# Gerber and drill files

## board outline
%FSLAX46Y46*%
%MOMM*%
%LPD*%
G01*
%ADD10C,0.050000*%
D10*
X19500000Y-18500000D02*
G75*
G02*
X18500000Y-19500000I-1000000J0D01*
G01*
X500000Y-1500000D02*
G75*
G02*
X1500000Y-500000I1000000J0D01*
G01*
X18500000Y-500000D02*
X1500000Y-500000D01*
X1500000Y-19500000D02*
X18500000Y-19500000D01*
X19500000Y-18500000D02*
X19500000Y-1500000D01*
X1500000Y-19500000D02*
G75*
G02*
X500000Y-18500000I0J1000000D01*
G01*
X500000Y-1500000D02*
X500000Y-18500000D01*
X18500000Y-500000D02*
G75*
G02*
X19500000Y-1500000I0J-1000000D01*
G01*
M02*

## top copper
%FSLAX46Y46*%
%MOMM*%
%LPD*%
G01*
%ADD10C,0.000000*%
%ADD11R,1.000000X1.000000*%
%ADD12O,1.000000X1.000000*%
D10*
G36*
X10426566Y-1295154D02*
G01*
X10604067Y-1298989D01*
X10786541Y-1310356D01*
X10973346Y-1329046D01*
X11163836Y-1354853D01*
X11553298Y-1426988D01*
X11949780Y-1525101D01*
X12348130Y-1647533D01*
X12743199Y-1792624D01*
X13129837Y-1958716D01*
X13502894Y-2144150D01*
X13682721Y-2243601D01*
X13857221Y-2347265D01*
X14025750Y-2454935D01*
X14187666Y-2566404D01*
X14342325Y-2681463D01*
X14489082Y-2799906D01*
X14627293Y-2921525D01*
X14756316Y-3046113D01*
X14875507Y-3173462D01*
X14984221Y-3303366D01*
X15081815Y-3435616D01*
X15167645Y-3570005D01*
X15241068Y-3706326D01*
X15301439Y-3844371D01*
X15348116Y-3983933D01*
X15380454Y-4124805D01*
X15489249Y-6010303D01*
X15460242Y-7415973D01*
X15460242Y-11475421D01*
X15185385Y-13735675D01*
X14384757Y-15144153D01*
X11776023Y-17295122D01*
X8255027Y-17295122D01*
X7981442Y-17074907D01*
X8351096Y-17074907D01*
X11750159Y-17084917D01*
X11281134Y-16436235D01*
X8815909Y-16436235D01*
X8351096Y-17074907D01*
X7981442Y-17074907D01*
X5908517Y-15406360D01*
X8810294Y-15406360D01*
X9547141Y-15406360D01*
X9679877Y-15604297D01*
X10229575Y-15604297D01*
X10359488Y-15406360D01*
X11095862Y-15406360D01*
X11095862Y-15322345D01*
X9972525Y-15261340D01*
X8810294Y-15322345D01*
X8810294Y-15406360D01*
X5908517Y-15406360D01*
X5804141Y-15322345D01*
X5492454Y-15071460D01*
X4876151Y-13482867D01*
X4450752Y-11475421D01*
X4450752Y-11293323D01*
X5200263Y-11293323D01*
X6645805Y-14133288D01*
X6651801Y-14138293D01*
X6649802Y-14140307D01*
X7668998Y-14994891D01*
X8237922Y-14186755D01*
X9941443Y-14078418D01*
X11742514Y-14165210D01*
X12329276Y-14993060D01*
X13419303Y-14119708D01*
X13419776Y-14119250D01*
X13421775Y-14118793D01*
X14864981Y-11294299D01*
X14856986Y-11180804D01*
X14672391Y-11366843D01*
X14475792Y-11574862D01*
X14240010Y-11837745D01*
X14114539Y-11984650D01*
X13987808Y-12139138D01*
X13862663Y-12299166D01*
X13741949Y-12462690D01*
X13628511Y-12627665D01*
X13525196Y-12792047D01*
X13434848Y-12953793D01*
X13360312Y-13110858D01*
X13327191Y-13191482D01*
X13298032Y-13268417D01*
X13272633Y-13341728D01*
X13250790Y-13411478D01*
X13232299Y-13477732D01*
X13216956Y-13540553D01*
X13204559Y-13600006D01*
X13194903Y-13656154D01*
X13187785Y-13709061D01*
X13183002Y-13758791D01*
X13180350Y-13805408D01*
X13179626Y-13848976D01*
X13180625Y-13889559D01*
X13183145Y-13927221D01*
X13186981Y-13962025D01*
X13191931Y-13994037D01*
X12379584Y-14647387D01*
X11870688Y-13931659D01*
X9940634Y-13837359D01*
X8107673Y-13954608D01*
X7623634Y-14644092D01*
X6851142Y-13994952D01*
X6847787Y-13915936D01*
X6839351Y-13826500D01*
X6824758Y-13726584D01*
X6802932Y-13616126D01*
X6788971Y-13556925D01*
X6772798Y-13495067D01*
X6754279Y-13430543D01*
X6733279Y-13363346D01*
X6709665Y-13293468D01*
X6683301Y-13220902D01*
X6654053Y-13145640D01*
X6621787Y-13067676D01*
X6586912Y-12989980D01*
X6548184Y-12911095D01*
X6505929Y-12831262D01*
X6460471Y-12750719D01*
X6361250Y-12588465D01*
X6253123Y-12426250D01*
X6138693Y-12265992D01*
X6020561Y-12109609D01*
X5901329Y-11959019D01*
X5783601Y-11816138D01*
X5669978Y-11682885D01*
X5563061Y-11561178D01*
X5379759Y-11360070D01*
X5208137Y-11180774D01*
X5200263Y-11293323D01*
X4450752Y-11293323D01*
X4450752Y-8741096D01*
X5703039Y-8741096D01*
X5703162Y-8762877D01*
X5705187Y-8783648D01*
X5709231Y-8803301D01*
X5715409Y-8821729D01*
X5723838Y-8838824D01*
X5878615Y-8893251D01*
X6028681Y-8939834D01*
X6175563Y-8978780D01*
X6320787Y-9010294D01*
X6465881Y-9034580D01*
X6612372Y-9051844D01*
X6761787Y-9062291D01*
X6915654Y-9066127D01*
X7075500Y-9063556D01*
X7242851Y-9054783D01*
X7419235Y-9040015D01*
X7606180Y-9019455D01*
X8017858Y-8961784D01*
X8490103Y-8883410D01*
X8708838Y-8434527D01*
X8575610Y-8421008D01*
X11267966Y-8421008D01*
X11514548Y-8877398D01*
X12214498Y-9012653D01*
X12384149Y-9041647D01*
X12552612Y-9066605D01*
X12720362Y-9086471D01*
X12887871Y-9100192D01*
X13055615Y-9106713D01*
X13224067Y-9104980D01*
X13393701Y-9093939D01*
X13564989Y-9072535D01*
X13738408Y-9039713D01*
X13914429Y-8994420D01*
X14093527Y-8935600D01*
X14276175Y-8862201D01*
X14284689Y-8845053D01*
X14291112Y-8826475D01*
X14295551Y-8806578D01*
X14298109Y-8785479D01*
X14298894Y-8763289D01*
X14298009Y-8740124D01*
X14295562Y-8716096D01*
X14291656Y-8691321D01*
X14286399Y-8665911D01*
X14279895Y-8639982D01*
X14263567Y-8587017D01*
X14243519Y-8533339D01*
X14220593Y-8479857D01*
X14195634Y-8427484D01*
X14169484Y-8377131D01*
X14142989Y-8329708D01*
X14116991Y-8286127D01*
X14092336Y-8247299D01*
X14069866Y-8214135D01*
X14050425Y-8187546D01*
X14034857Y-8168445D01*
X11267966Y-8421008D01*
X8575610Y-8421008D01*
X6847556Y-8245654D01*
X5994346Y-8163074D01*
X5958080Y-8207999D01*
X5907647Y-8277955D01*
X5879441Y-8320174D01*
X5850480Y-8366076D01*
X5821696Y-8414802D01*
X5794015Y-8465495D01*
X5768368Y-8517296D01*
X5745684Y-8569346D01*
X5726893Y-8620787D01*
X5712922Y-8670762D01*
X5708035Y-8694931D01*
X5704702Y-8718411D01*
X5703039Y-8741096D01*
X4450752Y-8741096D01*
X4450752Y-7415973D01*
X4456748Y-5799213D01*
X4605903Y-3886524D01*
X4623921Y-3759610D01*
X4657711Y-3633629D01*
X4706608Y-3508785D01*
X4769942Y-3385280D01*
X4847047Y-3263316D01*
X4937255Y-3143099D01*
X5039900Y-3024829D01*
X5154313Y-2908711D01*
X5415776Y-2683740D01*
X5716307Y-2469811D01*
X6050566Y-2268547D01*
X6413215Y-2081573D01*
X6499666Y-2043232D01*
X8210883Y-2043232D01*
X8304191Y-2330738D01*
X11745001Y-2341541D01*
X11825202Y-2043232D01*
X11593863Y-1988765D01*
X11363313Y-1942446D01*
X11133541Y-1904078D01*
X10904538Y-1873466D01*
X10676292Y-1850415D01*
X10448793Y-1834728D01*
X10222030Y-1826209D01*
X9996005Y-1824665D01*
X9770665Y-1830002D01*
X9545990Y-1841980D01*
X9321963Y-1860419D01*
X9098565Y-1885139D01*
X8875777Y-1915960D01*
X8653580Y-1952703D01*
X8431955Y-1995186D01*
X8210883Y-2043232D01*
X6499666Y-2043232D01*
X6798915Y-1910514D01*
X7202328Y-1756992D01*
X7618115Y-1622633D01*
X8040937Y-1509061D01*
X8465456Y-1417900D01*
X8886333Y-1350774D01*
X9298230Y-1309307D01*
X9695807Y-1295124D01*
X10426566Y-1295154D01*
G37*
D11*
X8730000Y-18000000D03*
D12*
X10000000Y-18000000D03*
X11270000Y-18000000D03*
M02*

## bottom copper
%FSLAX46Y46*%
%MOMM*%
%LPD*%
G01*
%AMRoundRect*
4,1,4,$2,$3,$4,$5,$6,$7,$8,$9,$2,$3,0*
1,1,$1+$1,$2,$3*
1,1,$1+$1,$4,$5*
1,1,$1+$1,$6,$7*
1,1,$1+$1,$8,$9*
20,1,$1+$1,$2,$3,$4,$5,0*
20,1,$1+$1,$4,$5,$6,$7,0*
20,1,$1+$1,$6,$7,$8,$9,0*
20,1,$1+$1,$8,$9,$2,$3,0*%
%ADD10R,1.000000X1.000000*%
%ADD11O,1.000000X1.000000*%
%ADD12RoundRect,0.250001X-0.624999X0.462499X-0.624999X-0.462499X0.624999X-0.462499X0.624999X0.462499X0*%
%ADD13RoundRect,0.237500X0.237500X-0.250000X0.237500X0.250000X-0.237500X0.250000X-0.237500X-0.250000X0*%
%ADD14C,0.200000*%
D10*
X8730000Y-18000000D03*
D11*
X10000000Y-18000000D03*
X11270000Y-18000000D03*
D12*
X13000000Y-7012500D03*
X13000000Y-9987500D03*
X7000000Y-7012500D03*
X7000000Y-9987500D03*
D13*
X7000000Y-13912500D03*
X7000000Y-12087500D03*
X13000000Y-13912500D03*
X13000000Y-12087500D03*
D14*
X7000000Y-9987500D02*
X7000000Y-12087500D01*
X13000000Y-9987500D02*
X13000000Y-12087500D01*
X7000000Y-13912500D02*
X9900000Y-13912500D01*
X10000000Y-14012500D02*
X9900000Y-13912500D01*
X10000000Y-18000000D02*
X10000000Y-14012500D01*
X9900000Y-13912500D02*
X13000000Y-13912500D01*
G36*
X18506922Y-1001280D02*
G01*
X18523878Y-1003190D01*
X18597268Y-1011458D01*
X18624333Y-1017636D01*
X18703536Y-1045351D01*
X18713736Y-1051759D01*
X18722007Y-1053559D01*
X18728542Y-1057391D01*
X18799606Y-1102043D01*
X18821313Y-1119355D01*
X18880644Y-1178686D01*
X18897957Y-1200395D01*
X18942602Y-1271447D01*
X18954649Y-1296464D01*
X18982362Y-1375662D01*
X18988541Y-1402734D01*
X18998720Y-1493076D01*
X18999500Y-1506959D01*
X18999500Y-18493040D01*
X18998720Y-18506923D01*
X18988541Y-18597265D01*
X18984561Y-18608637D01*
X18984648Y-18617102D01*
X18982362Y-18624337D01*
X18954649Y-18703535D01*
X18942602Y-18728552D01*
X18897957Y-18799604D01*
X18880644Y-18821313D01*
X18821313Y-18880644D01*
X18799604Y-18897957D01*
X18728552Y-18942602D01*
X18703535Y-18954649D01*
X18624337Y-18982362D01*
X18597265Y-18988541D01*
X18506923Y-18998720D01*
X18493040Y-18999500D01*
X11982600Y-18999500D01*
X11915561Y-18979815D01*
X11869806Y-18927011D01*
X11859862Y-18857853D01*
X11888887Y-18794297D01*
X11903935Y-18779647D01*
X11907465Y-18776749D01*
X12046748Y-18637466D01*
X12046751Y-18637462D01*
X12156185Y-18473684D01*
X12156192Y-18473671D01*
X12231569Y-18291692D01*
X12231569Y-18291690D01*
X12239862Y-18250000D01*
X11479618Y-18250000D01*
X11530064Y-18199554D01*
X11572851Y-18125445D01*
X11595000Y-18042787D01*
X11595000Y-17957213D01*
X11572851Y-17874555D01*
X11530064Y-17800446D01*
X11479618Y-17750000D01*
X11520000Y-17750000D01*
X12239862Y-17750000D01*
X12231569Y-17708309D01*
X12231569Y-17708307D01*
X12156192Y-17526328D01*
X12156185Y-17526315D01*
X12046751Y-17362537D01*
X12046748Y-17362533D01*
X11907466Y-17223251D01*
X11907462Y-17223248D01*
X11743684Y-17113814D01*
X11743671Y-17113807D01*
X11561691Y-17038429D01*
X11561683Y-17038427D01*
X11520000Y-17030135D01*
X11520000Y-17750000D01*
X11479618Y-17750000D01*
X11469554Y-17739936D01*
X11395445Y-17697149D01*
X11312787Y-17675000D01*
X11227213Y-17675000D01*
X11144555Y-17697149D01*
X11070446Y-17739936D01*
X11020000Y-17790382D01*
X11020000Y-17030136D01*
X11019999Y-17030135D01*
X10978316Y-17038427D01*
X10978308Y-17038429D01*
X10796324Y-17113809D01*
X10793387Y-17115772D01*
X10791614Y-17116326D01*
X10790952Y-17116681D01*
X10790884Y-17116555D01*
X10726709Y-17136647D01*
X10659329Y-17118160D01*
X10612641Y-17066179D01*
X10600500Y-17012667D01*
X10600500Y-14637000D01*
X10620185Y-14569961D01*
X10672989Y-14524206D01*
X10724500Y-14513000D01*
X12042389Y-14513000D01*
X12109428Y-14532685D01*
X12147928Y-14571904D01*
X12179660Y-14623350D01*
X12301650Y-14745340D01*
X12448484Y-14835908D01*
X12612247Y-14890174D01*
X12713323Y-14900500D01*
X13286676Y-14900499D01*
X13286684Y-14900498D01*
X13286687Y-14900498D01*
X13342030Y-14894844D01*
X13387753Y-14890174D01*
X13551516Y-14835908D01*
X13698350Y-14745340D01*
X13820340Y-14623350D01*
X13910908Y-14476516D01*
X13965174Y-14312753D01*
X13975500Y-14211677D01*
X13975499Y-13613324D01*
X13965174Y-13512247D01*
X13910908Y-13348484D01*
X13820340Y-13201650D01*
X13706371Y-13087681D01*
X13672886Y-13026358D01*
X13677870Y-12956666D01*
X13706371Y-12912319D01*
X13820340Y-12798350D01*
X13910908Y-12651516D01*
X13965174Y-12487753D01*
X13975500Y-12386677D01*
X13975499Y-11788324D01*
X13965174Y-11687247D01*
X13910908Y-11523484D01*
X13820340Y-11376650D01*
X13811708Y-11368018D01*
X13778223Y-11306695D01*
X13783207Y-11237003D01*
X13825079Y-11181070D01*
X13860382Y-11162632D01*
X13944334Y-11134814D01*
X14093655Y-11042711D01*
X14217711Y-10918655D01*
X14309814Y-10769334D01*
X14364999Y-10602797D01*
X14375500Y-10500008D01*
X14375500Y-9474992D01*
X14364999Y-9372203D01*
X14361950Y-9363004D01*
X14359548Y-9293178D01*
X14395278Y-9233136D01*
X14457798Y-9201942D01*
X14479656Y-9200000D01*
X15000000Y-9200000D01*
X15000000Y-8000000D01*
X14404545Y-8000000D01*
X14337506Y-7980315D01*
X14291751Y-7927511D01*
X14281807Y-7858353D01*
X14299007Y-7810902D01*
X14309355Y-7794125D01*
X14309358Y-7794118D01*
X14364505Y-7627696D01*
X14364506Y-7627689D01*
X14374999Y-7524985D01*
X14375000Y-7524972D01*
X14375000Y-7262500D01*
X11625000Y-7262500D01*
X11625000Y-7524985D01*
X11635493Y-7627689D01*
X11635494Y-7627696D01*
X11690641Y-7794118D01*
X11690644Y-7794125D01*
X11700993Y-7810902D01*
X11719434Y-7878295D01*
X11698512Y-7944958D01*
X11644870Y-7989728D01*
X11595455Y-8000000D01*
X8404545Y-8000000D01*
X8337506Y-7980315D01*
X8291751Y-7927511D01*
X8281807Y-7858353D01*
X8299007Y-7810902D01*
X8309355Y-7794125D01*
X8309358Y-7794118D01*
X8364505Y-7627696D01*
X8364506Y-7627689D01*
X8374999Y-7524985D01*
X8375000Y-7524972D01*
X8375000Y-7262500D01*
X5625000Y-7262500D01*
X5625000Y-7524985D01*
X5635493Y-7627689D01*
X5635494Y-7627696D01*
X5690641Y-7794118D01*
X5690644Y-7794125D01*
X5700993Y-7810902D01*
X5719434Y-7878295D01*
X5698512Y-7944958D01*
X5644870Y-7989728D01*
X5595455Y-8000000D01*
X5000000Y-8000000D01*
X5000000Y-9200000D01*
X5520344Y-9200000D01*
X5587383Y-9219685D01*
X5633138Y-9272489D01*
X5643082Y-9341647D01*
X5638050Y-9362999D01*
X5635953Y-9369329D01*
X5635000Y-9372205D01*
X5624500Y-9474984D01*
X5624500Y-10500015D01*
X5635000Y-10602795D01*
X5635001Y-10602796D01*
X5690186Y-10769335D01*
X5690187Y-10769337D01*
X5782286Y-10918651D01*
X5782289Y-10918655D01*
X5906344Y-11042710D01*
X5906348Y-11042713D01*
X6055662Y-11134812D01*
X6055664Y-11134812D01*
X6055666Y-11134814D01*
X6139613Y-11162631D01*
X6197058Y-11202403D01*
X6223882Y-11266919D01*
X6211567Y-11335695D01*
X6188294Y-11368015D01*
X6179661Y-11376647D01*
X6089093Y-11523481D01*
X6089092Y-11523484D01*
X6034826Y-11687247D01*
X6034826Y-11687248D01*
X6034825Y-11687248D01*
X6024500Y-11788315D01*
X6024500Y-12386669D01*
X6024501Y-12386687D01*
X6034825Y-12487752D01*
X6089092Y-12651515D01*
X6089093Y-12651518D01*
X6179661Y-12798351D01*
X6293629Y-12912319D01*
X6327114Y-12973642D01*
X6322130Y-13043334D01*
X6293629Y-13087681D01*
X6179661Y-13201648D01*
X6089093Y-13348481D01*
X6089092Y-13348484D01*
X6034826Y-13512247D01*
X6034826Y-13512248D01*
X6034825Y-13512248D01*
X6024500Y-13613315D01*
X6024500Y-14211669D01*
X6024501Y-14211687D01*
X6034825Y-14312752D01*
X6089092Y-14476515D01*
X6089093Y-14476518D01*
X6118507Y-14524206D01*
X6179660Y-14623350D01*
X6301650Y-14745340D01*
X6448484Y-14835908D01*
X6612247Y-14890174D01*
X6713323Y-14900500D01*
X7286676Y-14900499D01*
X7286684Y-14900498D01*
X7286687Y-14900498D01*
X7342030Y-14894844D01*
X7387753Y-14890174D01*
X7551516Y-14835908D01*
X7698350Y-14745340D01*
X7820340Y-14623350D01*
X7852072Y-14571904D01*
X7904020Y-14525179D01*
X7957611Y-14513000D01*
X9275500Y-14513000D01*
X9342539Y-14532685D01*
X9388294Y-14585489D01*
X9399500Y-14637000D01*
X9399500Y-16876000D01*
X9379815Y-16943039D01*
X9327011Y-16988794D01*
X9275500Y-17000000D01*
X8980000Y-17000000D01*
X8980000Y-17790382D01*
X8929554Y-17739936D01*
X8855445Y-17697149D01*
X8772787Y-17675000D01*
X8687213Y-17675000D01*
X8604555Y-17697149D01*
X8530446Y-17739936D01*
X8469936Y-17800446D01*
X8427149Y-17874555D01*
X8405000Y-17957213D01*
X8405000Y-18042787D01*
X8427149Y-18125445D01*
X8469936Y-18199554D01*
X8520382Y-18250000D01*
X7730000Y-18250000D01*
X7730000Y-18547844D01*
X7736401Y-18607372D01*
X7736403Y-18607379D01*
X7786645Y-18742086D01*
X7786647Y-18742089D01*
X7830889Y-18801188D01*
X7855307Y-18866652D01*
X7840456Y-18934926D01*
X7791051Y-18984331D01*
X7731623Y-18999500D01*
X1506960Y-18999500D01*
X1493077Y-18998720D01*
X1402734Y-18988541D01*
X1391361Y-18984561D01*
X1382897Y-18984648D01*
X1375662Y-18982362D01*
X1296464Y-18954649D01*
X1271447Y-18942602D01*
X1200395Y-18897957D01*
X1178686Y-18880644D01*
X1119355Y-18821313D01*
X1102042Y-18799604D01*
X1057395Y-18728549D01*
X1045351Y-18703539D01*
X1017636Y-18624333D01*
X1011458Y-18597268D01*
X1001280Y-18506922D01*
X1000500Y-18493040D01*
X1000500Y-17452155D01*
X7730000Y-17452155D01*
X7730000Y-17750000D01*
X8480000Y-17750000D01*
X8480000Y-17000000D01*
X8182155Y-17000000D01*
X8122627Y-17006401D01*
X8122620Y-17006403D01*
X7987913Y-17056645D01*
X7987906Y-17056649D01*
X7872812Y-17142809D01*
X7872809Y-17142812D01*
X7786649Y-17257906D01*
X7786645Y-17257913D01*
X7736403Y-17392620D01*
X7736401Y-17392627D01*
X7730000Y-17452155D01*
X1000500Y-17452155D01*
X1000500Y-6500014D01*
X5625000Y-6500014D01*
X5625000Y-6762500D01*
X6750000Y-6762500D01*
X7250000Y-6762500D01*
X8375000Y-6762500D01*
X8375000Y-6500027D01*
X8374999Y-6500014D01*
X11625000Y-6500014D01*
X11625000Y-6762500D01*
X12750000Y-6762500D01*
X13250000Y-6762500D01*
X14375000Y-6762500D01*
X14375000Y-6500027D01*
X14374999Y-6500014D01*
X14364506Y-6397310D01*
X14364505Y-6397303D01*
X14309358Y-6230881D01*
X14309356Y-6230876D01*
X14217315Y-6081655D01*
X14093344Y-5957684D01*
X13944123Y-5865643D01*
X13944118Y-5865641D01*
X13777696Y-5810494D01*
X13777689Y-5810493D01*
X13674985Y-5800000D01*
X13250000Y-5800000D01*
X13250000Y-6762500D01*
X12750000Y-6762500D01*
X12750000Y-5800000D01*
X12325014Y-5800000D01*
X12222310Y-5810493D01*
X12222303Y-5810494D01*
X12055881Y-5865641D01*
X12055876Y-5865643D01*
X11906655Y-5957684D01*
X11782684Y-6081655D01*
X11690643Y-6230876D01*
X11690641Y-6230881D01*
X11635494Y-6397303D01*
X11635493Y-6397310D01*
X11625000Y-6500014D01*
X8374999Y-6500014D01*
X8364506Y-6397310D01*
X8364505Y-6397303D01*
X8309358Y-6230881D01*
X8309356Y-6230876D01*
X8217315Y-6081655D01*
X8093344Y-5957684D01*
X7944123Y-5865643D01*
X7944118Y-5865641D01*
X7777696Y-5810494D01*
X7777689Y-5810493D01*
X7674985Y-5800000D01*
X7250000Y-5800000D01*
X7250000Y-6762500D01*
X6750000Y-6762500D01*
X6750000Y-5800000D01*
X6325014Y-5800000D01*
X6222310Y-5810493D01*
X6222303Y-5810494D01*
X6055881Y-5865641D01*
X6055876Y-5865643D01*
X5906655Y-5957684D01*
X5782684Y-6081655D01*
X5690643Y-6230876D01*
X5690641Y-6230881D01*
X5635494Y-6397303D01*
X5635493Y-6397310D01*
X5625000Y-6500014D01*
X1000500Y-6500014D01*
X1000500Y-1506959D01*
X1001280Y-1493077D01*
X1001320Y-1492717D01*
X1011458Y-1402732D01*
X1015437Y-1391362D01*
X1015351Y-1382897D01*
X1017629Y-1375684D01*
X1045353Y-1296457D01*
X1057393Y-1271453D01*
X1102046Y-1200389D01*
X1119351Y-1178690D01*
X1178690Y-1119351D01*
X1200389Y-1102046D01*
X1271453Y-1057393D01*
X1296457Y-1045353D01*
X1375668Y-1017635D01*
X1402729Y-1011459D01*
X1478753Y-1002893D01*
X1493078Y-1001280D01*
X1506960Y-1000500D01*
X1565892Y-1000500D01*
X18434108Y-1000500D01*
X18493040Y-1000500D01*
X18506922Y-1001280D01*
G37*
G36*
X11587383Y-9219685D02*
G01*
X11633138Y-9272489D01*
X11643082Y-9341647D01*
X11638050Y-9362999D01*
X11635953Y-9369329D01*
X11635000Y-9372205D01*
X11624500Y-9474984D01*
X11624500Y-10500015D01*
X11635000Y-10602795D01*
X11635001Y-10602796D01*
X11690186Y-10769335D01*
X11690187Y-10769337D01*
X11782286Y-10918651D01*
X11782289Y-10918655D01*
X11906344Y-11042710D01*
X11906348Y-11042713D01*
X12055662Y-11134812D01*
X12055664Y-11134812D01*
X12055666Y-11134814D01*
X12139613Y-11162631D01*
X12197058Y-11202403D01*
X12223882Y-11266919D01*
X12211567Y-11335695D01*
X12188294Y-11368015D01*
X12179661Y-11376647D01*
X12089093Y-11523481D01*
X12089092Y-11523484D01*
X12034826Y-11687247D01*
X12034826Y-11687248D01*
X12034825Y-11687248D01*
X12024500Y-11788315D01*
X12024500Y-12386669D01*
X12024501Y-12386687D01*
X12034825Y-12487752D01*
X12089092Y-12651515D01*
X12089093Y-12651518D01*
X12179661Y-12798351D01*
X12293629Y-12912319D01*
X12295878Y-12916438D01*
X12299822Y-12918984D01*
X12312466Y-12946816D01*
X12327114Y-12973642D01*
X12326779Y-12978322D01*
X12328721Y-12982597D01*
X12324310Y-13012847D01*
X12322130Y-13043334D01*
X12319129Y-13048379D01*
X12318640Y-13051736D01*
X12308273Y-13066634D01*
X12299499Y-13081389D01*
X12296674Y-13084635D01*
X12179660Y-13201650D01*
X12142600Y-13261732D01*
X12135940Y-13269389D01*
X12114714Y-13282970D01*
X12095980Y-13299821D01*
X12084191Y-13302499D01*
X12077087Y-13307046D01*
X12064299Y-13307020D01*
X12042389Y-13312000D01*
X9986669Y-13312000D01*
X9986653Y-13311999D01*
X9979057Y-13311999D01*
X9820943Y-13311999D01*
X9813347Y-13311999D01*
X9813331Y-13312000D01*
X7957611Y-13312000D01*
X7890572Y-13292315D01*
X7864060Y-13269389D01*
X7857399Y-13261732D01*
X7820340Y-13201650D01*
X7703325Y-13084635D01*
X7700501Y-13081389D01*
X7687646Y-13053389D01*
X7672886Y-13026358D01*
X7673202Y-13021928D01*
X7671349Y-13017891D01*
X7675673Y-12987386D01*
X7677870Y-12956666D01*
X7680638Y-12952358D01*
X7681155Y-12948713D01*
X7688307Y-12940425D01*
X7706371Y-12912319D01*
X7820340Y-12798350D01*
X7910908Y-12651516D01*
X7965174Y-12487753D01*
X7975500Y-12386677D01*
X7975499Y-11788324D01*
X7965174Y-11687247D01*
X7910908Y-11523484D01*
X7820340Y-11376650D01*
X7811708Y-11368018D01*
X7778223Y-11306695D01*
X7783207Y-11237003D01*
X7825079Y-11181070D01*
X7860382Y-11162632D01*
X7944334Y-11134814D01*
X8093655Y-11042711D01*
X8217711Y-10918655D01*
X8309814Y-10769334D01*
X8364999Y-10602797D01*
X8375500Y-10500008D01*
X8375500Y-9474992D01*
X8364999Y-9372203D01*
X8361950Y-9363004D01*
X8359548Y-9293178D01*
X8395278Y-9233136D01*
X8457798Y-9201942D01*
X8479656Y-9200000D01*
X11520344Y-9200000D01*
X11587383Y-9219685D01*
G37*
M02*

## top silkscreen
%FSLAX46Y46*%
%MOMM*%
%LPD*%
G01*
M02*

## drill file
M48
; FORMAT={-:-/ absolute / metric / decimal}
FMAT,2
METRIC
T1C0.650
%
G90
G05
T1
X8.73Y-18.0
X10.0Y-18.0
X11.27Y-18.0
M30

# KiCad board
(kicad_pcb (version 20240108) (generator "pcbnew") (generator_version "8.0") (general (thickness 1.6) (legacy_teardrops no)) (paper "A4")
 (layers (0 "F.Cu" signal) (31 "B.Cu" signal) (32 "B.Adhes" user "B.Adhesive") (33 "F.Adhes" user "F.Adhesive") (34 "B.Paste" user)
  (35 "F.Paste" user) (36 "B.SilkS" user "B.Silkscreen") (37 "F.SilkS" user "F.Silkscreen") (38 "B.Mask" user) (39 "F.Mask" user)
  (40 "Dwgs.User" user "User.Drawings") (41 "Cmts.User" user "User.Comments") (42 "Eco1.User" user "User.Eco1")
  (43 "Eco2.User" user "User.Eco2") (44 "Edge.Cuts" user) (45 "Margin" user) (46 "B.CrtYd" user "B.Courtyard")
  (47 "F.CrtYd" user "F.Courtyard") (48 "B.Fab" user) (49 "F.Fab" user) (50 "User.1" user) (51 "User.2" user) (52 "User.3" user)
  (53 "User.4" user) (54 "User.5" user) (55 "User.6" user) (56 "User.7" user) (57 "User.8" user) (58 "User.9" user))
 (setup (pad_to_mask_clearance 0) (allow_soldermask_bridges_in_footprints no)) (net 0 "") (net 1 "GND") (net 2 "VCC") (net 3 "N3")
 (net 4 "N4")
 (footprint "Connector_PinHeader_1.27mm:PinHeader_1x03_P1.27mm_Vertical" (layer "B.Cu") (at 8.73 18 -90)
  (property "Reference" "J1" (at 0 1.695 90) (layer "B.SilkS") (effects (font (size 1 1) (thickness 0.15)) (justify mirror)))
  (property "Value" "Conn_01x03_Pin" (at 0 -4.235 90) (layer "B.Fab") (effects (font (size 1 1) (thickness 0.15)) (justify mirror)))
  (pad "1" thru_hole rect (at 0 0 270) (size 1 1) (drill 0.65) (layers "*.Cu" "*.Mask") (remove_unused_layers no) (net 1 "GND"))
  (pad "2" thru_hole oval (at 0 -1.27 270) (size 1 1) (drill 0.65) (layers "*.Cu" "*.Mask") (remove_unused_layers no) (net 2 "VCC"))
  (pad "3" thru_hole oval (at 0 -2.54 270) (size 1 1) (drill 0.65) (layers "*.Cu" "*.Mask") (remove_unused_layers no) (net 1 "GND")))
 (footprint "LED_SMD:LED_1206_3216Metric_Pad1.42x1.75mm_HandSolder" (layer "B.Cu") (at 13 8.5 -90)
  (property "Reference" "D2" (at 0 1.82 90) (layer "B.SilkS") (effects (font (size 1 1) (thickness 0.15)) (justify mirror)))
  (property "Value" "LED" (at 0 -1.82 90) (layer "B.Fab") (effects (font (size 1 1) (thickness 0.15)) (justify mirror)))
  (pad "1" smd roundrect (at -1.4875 0 270) (size 1.425 1.75) (layers "B.Cu" "B.Paste" "B.Mask") (roundrect_rratio 0.175439) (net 1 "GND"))
  (pad "2" smd roundrect (at 1.4875 0 270) (size 1.425 1.75) (layers "B.Cu" "B.Paste" "B.Mask") (roundrect_rratio 0.175439) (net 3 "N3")))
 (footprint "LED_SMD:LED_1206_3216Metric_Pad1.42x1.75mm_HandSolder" (layer "B.Cu") (at 7 8.5 -90)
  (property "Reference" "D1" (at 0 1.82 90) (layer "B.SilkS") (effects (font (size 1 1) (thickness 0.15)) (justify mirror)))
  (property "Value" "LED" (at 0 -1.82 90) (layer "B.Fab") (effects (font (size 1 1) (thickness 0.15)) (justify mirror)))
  (pad "1" smd roundrect (at -1.4875 0 270) (size 1.425 1.75) (layers "B.Cu" "B.Paste" "B.Mask") (roundrect_rratio 0.175439) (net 1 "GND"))
  (pad "2" smd roundrect (at 1.4875 0 270) (size 1.425 1.75) (layers "B.Cu" "B.Paste" "B.Mask") (roundrect_rratio 0.175439) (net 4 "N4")))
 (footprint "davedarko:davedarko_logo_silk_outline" (layer "B.Cu") (at 16.4 15.9 180)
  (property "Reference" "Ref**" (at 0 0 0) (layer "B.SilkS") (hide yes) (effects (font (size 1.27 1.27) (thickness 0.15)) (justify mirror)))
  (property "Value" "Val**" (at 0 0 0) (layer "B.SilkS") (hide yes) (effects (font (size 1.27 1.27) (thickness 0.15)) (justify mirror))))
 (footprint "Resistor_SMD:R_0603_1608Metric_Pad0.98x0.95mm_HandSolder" (layer "B.Cu") (at 7 13 90)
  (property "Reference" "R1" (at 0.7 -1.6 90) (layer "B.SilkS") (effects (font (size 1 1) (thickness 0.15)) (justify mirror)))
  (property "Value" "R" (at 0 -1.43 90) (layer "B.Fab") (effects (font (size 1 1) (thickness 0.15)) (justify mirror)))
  (pad "1" smd roundrect (at -0.9125 0 90) (size 0.975 0.95) (layers "B.Cu" "B.Paste" "B.Mask") (roundrect_rratio 0.25) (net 2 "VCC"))
  (pad "2" smd roundrect (at 0.9125 0 90) (size 0.975 0.95) (layers "B.Cu" "B.Paste" "B.Mask") (roundrect_rratio 0.25) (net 4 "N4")))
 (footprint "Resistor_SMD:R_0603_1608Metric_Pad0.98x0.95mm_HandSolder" (layer "B.Cu") (at 13 13 90)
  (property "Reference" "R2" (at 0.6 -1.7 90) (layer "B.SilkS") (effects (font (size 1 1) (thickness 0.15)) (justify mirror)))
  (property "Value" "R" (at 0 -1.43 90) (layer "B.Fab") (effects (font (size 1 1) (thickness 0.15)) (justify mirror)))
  (pad "1" smd roundrect (at -0.9125 0 90) (size 0.975 0.95) (layers "B.Cu" "B.Paste" "B.Mask") (roundrect_rratio 0.25) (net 2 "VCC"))
  (pad "2" smd roundrect (at 0.9125 0 90) (size 0.975 0.95) (layers "B.Cu" "B.Paste" "B.Mask") (roundrect_rratio 0.25) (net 3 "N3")))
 (gr_poly
  (pts (xy 10.426566 1.295154) (xy 10.604067 1.298989) (xy 10.786541 1.310356) (xy 10.973346 1.329046) (xy 11.163836 1.354853)
   (xy 11.553298 1.426988) (xy 11.94978 1.525101) (xy 12.34813 1.647533) (xy 12.743199 1.792624) (xy 13.129837 1.958716)
   (xy 13.502894 2.14415) (xy 13.682721 2.243601) (xy 13.857221 2.347265) (xy 14.02575 2.454935) (xy 14.187666 2.566404)
   (xy 14.342325 2.681463) (xy 14.489082 2.799906) (xy 14.627293 2.921525) (xy 14.756316 3.046113) (xy 14.875507 3.173462)
   (xy 14.984221 3.303366) (xy 15.081815 3.435616) (xy 15.167645 3.570005) (xy 15.241068 3.706326) (xy 15.301439 3.844371)
   (xy 15.348116 3.983933) (xy 15.380454 4.124805) (xy 15.489249 6.010303) (xy 15.460242 7.415973) (xy 15.460242 11.475421)
   (xy 15.185385 13.735675) (xy 14.384757 15.144153) (xy 11.776023 17.295122) (xy 8.255027 17.295122) (xy 7.981442 17.074907)
   (xy 8.351096 17.074907) (xy 11.750159 17.084917) (xy 11.281134 16.436235) (xy 8.815909 16.436235) (xy 8.351096 17.074907)
   (xy 7.981442 17.074907) (xy 5.804141 15.322345) (xy 8.810294 15.322345) (xy 8.810294 15.40636) (xy 9.547141 15.40636)
   (xy 9.679877 15.604297) (xy 10.229575 15.604297) (xy 10.359488 15.40636) (xy 11.095862 15.40636) (xy 11.095862 15.322345)
   (xy 9.972525 15.26134) (xy 8.810294 15.322345) (xy 5.804141 15.322345) (xy 5.492454 15.07146) (xy 4.876151 13.482867)
   (xy 4.450752 11.475421) (xy 4.450752 11.293323) (xy 5.200263 11.293323) (xy 6.645805 14.133288) (xy 6.651801 14.138293)
   (xy 6.649802 14.140307) (xy 7.668998 14.994891) (xy 8.237922 14.186755) (xy 9.941443 14.078418) (xy 11.742514 14.16521)
   (xy 12.329276 14.99306) (xy 13.419303 14.119708) (xy 13.419776 14.11925) (xy 13.421775 14.118793) (xy 14.864981 11.294299)
   (xy 14.856986 11.180804) (xy 14.672391 11.366843) (xy 14.475792 11.574862) (xy 14.24001 11.837745) (xy 14.114539 11.98465)
   (xy 13.987808 12.139138) (xy 13.862663 12.299166) (xy 13.741949 12.46269) (xy 13.628511 12.627665) (xy 13.525196 12.792047)
   (xy 13.434848 12.953793) (xy 13.360312 13.110858) (xy 13.327191 13.191482) (xy 13.298032 13.268417) (xy 13.272633 13.341728)
   (xy 13.25079 13.411478) (xy 13.232299 13.477732) (xy 13.216956 13.540553) (xy 13.204559 13.600006) (xy 13.194903 13.656154)
   (xy 13.187785 13.709061) (xy 13.183002 13.758791) (xy 13.18035 13.805408) (xy 13.179626 13.848976) (xy 13.180625 13.889559)
   (xy 13.183145 13.927221) (xy 13.186981 13.962025) (xy 13.191931 13.994037) (xy 12.379584 14.647387) (xy 11.870688 13.931659)
   (xy 9.940634 13.837359) (xy 8.107673 13.954608) (xy 7.623634 14.644092) (xy 6.851142 13.994952) (xy 6.847787 13.915936)
   (xy 6.839351 13.8265) (xy 6.824758 13.726584) (xy 6.802932 13.616126) (xy 6.788971 13.556925) (xy 6.772798 13.495067)
   (xy 6.754279 13.430543) (xy 6.733279 13.363346) (xy 6.709665 13.293468) (xy 6.683301 13.220902) (xy 6.654053 13.14564)
   (xy 6.621787 13.067676) (xy 6.586912 12.98998) (xy 6.548184 12.911095) (xy 6.505929 12.831262) (xy 6.460471 12.750719)
   (xy 6.36125 12.588465) (xy 6.253123 12.42625) (xy 6.138693 12.265992) (xy 6.020561 12.109609) (xy 5.901329 11.959019)
   (xy 5.783601 11.816138) (xy 5.669978 11.682885) (xy 5.563061 11.561178) (xy 5.379759 11.36007) (xy 5.208137 11.180774)
   (xy 5.200263 11.293323) (xy 4.450752 11.293323) (xy 4.450752 8.741096) (xy 5.703039 8.741096) (xy 5.703162 8.762877)
   (xy 5.705187 8.783648) (xy 5.709231 8.803301) (xy 5.715409 8.821729) (xy 5.723838 8.838824) (xy 5.878615 8.893251) (xy 6.028681 8.939834)
   (xy 6.175563 8.97878) (xy 6.320787 9.010294) (xy 6.465881 9.03458) (xy 6.612372 9.051844) (xy 6.761787 9.062291) (xy 6.915654 9.066127)
   (xy 7.0755 9.063556) (xy 7.242851 9.054783) (xy 7.419235 9.040015) (xy 7.60618 9.019455) (xy 8.017858 8.961784) (xy 8.490103 8.88341)
   (xy 8.708838 8.434527) (xy 8.57561 8.421008) (xy 11.267966 8.421008) (xy 11.514548 8.877398) (xy 12.214498 9.012653)
   (xy 12.384149 9.041647) (xy 12.552612 9.066605) (xy 12.720362 9.086471) (xy 12.887871 9.100192) (xy 13.055615 9.106713)
   (xy 13.224067 9.10498) (xy 13.393701 9.093939) (xy 13.564989 9.072535) (xy 13.738408 9.039713) (xy 13.914429 8.99442)
   (xy 14.093527 8.9356) (xy 14.276175 8.862201) (xy 14.284689 8.845053) (xy 14.291112 8.826475) (xy 14.295551 8.806578)
   (xy 14.298109 8.785479) (xy 14.298894 8.763289) (xy 14.298009 8.740124) (xy 14.295562 8.716096) (xy 14.291656 8.691321)
   (xy 14.286399 8.665911) (xy 14.279895 8.639982) (xy 14.263567 8.587017) (xy 14.243519 8.533339) (xy 14.220593 8.479857)
   (xy 14.195634 8.427484) (xy 14.169484 8.377131) (xy 14.142989 8.329708) (xy 14.116991 8.286127) (xy 14.092336 8.247299)
   (xy 14.069866 8.214135) (xy 14.050425 8.187546) (xy 14.034857 8.168445) (xy 11.267966 8.421008) (xy 8.57561 8.421008)
   (xy 6.847556 8.245654) (xy 5.994346 8.163074) (xy 5.95808 8.207999) (xy 5.907647 8.277955) (xy 5.879441 8.320174) (xy 5.85048 8.366076)
   (xy 5.821696 8.414802) (xy 5.794015 8.465495) (xy 5.768368 8.517296) (xy 5.745684 8.569346) (xy 5.726893 8.620787) (xy 5.712922 8.670762)
   (xy 5.708035 8.694931) (xy 5.704702 8.718411) (xy 5.703039 8.741096) (xy 4.450752 8.741096) (xy 4.450752 7.415973) (xy 4.456748 5.799213)
   (xy 4.605903 3.886524) (xy 4.623921 3.75961) (xy 4.657711 3.633629) (xy 4.706608 3.508785) (xy 4.769942 3.38528) (xy 4.847047 3.263316)
   (xy 4.937255 3.143099) (xy 5.0399 3.024829) (xy 5.154313 2.908711) (xy 5.415776 2.68374) (xy 5.716307 2.469811) (xy 6.050566 2.268547)
   (xy 6.413215 2.081573) (xy 6.499666 2.043232) (xy 8.210883 2.043232) (xy 8.304191 2.330738) (xy 11.745001 2.341541)
   (xy 11.825202 2.043232) (xy 11.593863 1.988765) (xy 11.363313 1.942446) (xy 11.133541 1.904078) (xy 10.904538 1.873466)
   (xy 10.676292 1.850415) (xy 10.448793 1.834728) (xy 10.22203 1.826209) (xy 9.996005 1.824665) (xy 9.770665 1.830002) (xy 9.54599 1.84198)
   (xy 9.321963 1.860419) (xy 9.098565 1.885139) (xy 8.875777 1.91596) (xy 8.65358 1.952703) (xy 8.431955 1.995186) (xy 8.210883 2.043232)
   (xy 6.499666 2.043232) (xy 6.798915 1.910514) (xy 7.202328 1.756992) (xy 7.618115 1.622633) (xy 8.040937 1.509061) (xy 8.465456 1.4179)
   (xy 8.886333 1.350774) (xy 9.29823 1.309307) (xy 9.695807 1.295124))
  (stroke (width -0.000001) (type solid)) (fill solid) (layer "F.Cu"))
 (gr_arc (start 19.5 18.5) (mid 19.207107 19.207107) (end 18.5 19.5) (stroke (width 0.05) (type default)) (layer "Edge.Cuts"))
 (gr_arc (start 0.5 1.5) (mid 0.792893 0.792893) (end 1.5 0.5) (stroke (width 0.05) (type default)) (layer "Edge.Cuts"))
 (gr_line (start 18.5 0.5) (end 1.5 0.5) (stroke (width 0.05) (type default)) (layer "Edge.Cuts"))
 (gr_line (start 1.5 19.5) (end 18.5 19.5) (stroke (width 0.05) (type default)) (layer "Edge.Cuts"))
 (gr_line (start 19.5 18.5) (end 19.5 1.5) (stroke (width 0.05) (type default)) (layer "Edge.Cuts"))
 (gr_arc (start 1.5 19.5) (mid 0.792893 19.207107) (end 0.5 18.5) (stroke (width 0.05) (type default)) (layer "Edge.Cuts"))
 (gr_line (start 0.5 1.5) (end 0.5 18.5) (stroke (width 0.05) (type default)) (layer "Edge.Cuts"))
 (gr_arc (start 18.5 0.5) (mid 19.207107 0.792893) (end 19.5 1.5) (stroke (width 0.05) (type default)) (layer "Edge.Cuts"))
 (segment (start 7 9.9875) (end 7 12.0875) (width 0.2) (layer "B.Cu") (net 4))
 (segment (start 13 9.9875) (end 13 12.0875) (width 0.2) (layer "B.Cu") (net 3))
 (segment (start 7 13.9125) (end 9.9 13.9125) (width 0.2) (layer "B.Cu") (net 2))
 (segment (start 10 14.0125) (end 9.9 13.9125) (width 0.2) (layer "B.Cu") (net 2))
 (segment (start 10 18) (end 10 14.0125) (width 0.2) (layer "B.Cu") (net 2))
 (segment (start 9.9 13.9125) (end 13 13.9125) (width 0.2) (layer "B.Cu") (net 2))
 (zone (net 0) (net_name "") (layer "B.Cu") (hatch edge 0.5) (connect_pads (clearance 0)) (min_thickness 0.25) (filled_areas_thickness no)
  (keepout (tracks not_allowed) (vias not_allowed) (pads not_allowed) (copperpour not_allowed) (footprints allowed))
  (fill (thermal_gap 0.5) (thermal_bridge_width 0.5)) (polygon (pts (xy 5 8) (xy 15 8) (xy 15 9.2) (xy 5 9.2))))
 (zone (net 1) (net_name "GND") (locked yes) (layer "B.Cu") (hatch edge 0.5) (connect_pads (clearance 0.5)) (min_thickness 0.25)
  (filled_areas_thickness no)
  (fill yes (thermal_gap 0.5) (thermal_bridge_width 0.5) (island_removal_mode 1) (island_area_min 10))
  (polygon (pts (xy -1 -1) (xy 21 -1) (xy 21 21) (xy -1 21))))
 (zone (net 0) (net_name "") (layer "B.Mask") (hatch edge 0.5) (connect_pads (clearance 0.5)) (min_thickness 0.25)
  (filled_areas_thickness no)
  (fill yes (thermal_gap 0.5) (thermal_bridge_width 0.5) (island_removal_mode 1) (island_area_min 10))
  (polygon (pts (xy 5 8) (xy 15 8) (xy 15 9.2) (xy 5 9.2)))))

